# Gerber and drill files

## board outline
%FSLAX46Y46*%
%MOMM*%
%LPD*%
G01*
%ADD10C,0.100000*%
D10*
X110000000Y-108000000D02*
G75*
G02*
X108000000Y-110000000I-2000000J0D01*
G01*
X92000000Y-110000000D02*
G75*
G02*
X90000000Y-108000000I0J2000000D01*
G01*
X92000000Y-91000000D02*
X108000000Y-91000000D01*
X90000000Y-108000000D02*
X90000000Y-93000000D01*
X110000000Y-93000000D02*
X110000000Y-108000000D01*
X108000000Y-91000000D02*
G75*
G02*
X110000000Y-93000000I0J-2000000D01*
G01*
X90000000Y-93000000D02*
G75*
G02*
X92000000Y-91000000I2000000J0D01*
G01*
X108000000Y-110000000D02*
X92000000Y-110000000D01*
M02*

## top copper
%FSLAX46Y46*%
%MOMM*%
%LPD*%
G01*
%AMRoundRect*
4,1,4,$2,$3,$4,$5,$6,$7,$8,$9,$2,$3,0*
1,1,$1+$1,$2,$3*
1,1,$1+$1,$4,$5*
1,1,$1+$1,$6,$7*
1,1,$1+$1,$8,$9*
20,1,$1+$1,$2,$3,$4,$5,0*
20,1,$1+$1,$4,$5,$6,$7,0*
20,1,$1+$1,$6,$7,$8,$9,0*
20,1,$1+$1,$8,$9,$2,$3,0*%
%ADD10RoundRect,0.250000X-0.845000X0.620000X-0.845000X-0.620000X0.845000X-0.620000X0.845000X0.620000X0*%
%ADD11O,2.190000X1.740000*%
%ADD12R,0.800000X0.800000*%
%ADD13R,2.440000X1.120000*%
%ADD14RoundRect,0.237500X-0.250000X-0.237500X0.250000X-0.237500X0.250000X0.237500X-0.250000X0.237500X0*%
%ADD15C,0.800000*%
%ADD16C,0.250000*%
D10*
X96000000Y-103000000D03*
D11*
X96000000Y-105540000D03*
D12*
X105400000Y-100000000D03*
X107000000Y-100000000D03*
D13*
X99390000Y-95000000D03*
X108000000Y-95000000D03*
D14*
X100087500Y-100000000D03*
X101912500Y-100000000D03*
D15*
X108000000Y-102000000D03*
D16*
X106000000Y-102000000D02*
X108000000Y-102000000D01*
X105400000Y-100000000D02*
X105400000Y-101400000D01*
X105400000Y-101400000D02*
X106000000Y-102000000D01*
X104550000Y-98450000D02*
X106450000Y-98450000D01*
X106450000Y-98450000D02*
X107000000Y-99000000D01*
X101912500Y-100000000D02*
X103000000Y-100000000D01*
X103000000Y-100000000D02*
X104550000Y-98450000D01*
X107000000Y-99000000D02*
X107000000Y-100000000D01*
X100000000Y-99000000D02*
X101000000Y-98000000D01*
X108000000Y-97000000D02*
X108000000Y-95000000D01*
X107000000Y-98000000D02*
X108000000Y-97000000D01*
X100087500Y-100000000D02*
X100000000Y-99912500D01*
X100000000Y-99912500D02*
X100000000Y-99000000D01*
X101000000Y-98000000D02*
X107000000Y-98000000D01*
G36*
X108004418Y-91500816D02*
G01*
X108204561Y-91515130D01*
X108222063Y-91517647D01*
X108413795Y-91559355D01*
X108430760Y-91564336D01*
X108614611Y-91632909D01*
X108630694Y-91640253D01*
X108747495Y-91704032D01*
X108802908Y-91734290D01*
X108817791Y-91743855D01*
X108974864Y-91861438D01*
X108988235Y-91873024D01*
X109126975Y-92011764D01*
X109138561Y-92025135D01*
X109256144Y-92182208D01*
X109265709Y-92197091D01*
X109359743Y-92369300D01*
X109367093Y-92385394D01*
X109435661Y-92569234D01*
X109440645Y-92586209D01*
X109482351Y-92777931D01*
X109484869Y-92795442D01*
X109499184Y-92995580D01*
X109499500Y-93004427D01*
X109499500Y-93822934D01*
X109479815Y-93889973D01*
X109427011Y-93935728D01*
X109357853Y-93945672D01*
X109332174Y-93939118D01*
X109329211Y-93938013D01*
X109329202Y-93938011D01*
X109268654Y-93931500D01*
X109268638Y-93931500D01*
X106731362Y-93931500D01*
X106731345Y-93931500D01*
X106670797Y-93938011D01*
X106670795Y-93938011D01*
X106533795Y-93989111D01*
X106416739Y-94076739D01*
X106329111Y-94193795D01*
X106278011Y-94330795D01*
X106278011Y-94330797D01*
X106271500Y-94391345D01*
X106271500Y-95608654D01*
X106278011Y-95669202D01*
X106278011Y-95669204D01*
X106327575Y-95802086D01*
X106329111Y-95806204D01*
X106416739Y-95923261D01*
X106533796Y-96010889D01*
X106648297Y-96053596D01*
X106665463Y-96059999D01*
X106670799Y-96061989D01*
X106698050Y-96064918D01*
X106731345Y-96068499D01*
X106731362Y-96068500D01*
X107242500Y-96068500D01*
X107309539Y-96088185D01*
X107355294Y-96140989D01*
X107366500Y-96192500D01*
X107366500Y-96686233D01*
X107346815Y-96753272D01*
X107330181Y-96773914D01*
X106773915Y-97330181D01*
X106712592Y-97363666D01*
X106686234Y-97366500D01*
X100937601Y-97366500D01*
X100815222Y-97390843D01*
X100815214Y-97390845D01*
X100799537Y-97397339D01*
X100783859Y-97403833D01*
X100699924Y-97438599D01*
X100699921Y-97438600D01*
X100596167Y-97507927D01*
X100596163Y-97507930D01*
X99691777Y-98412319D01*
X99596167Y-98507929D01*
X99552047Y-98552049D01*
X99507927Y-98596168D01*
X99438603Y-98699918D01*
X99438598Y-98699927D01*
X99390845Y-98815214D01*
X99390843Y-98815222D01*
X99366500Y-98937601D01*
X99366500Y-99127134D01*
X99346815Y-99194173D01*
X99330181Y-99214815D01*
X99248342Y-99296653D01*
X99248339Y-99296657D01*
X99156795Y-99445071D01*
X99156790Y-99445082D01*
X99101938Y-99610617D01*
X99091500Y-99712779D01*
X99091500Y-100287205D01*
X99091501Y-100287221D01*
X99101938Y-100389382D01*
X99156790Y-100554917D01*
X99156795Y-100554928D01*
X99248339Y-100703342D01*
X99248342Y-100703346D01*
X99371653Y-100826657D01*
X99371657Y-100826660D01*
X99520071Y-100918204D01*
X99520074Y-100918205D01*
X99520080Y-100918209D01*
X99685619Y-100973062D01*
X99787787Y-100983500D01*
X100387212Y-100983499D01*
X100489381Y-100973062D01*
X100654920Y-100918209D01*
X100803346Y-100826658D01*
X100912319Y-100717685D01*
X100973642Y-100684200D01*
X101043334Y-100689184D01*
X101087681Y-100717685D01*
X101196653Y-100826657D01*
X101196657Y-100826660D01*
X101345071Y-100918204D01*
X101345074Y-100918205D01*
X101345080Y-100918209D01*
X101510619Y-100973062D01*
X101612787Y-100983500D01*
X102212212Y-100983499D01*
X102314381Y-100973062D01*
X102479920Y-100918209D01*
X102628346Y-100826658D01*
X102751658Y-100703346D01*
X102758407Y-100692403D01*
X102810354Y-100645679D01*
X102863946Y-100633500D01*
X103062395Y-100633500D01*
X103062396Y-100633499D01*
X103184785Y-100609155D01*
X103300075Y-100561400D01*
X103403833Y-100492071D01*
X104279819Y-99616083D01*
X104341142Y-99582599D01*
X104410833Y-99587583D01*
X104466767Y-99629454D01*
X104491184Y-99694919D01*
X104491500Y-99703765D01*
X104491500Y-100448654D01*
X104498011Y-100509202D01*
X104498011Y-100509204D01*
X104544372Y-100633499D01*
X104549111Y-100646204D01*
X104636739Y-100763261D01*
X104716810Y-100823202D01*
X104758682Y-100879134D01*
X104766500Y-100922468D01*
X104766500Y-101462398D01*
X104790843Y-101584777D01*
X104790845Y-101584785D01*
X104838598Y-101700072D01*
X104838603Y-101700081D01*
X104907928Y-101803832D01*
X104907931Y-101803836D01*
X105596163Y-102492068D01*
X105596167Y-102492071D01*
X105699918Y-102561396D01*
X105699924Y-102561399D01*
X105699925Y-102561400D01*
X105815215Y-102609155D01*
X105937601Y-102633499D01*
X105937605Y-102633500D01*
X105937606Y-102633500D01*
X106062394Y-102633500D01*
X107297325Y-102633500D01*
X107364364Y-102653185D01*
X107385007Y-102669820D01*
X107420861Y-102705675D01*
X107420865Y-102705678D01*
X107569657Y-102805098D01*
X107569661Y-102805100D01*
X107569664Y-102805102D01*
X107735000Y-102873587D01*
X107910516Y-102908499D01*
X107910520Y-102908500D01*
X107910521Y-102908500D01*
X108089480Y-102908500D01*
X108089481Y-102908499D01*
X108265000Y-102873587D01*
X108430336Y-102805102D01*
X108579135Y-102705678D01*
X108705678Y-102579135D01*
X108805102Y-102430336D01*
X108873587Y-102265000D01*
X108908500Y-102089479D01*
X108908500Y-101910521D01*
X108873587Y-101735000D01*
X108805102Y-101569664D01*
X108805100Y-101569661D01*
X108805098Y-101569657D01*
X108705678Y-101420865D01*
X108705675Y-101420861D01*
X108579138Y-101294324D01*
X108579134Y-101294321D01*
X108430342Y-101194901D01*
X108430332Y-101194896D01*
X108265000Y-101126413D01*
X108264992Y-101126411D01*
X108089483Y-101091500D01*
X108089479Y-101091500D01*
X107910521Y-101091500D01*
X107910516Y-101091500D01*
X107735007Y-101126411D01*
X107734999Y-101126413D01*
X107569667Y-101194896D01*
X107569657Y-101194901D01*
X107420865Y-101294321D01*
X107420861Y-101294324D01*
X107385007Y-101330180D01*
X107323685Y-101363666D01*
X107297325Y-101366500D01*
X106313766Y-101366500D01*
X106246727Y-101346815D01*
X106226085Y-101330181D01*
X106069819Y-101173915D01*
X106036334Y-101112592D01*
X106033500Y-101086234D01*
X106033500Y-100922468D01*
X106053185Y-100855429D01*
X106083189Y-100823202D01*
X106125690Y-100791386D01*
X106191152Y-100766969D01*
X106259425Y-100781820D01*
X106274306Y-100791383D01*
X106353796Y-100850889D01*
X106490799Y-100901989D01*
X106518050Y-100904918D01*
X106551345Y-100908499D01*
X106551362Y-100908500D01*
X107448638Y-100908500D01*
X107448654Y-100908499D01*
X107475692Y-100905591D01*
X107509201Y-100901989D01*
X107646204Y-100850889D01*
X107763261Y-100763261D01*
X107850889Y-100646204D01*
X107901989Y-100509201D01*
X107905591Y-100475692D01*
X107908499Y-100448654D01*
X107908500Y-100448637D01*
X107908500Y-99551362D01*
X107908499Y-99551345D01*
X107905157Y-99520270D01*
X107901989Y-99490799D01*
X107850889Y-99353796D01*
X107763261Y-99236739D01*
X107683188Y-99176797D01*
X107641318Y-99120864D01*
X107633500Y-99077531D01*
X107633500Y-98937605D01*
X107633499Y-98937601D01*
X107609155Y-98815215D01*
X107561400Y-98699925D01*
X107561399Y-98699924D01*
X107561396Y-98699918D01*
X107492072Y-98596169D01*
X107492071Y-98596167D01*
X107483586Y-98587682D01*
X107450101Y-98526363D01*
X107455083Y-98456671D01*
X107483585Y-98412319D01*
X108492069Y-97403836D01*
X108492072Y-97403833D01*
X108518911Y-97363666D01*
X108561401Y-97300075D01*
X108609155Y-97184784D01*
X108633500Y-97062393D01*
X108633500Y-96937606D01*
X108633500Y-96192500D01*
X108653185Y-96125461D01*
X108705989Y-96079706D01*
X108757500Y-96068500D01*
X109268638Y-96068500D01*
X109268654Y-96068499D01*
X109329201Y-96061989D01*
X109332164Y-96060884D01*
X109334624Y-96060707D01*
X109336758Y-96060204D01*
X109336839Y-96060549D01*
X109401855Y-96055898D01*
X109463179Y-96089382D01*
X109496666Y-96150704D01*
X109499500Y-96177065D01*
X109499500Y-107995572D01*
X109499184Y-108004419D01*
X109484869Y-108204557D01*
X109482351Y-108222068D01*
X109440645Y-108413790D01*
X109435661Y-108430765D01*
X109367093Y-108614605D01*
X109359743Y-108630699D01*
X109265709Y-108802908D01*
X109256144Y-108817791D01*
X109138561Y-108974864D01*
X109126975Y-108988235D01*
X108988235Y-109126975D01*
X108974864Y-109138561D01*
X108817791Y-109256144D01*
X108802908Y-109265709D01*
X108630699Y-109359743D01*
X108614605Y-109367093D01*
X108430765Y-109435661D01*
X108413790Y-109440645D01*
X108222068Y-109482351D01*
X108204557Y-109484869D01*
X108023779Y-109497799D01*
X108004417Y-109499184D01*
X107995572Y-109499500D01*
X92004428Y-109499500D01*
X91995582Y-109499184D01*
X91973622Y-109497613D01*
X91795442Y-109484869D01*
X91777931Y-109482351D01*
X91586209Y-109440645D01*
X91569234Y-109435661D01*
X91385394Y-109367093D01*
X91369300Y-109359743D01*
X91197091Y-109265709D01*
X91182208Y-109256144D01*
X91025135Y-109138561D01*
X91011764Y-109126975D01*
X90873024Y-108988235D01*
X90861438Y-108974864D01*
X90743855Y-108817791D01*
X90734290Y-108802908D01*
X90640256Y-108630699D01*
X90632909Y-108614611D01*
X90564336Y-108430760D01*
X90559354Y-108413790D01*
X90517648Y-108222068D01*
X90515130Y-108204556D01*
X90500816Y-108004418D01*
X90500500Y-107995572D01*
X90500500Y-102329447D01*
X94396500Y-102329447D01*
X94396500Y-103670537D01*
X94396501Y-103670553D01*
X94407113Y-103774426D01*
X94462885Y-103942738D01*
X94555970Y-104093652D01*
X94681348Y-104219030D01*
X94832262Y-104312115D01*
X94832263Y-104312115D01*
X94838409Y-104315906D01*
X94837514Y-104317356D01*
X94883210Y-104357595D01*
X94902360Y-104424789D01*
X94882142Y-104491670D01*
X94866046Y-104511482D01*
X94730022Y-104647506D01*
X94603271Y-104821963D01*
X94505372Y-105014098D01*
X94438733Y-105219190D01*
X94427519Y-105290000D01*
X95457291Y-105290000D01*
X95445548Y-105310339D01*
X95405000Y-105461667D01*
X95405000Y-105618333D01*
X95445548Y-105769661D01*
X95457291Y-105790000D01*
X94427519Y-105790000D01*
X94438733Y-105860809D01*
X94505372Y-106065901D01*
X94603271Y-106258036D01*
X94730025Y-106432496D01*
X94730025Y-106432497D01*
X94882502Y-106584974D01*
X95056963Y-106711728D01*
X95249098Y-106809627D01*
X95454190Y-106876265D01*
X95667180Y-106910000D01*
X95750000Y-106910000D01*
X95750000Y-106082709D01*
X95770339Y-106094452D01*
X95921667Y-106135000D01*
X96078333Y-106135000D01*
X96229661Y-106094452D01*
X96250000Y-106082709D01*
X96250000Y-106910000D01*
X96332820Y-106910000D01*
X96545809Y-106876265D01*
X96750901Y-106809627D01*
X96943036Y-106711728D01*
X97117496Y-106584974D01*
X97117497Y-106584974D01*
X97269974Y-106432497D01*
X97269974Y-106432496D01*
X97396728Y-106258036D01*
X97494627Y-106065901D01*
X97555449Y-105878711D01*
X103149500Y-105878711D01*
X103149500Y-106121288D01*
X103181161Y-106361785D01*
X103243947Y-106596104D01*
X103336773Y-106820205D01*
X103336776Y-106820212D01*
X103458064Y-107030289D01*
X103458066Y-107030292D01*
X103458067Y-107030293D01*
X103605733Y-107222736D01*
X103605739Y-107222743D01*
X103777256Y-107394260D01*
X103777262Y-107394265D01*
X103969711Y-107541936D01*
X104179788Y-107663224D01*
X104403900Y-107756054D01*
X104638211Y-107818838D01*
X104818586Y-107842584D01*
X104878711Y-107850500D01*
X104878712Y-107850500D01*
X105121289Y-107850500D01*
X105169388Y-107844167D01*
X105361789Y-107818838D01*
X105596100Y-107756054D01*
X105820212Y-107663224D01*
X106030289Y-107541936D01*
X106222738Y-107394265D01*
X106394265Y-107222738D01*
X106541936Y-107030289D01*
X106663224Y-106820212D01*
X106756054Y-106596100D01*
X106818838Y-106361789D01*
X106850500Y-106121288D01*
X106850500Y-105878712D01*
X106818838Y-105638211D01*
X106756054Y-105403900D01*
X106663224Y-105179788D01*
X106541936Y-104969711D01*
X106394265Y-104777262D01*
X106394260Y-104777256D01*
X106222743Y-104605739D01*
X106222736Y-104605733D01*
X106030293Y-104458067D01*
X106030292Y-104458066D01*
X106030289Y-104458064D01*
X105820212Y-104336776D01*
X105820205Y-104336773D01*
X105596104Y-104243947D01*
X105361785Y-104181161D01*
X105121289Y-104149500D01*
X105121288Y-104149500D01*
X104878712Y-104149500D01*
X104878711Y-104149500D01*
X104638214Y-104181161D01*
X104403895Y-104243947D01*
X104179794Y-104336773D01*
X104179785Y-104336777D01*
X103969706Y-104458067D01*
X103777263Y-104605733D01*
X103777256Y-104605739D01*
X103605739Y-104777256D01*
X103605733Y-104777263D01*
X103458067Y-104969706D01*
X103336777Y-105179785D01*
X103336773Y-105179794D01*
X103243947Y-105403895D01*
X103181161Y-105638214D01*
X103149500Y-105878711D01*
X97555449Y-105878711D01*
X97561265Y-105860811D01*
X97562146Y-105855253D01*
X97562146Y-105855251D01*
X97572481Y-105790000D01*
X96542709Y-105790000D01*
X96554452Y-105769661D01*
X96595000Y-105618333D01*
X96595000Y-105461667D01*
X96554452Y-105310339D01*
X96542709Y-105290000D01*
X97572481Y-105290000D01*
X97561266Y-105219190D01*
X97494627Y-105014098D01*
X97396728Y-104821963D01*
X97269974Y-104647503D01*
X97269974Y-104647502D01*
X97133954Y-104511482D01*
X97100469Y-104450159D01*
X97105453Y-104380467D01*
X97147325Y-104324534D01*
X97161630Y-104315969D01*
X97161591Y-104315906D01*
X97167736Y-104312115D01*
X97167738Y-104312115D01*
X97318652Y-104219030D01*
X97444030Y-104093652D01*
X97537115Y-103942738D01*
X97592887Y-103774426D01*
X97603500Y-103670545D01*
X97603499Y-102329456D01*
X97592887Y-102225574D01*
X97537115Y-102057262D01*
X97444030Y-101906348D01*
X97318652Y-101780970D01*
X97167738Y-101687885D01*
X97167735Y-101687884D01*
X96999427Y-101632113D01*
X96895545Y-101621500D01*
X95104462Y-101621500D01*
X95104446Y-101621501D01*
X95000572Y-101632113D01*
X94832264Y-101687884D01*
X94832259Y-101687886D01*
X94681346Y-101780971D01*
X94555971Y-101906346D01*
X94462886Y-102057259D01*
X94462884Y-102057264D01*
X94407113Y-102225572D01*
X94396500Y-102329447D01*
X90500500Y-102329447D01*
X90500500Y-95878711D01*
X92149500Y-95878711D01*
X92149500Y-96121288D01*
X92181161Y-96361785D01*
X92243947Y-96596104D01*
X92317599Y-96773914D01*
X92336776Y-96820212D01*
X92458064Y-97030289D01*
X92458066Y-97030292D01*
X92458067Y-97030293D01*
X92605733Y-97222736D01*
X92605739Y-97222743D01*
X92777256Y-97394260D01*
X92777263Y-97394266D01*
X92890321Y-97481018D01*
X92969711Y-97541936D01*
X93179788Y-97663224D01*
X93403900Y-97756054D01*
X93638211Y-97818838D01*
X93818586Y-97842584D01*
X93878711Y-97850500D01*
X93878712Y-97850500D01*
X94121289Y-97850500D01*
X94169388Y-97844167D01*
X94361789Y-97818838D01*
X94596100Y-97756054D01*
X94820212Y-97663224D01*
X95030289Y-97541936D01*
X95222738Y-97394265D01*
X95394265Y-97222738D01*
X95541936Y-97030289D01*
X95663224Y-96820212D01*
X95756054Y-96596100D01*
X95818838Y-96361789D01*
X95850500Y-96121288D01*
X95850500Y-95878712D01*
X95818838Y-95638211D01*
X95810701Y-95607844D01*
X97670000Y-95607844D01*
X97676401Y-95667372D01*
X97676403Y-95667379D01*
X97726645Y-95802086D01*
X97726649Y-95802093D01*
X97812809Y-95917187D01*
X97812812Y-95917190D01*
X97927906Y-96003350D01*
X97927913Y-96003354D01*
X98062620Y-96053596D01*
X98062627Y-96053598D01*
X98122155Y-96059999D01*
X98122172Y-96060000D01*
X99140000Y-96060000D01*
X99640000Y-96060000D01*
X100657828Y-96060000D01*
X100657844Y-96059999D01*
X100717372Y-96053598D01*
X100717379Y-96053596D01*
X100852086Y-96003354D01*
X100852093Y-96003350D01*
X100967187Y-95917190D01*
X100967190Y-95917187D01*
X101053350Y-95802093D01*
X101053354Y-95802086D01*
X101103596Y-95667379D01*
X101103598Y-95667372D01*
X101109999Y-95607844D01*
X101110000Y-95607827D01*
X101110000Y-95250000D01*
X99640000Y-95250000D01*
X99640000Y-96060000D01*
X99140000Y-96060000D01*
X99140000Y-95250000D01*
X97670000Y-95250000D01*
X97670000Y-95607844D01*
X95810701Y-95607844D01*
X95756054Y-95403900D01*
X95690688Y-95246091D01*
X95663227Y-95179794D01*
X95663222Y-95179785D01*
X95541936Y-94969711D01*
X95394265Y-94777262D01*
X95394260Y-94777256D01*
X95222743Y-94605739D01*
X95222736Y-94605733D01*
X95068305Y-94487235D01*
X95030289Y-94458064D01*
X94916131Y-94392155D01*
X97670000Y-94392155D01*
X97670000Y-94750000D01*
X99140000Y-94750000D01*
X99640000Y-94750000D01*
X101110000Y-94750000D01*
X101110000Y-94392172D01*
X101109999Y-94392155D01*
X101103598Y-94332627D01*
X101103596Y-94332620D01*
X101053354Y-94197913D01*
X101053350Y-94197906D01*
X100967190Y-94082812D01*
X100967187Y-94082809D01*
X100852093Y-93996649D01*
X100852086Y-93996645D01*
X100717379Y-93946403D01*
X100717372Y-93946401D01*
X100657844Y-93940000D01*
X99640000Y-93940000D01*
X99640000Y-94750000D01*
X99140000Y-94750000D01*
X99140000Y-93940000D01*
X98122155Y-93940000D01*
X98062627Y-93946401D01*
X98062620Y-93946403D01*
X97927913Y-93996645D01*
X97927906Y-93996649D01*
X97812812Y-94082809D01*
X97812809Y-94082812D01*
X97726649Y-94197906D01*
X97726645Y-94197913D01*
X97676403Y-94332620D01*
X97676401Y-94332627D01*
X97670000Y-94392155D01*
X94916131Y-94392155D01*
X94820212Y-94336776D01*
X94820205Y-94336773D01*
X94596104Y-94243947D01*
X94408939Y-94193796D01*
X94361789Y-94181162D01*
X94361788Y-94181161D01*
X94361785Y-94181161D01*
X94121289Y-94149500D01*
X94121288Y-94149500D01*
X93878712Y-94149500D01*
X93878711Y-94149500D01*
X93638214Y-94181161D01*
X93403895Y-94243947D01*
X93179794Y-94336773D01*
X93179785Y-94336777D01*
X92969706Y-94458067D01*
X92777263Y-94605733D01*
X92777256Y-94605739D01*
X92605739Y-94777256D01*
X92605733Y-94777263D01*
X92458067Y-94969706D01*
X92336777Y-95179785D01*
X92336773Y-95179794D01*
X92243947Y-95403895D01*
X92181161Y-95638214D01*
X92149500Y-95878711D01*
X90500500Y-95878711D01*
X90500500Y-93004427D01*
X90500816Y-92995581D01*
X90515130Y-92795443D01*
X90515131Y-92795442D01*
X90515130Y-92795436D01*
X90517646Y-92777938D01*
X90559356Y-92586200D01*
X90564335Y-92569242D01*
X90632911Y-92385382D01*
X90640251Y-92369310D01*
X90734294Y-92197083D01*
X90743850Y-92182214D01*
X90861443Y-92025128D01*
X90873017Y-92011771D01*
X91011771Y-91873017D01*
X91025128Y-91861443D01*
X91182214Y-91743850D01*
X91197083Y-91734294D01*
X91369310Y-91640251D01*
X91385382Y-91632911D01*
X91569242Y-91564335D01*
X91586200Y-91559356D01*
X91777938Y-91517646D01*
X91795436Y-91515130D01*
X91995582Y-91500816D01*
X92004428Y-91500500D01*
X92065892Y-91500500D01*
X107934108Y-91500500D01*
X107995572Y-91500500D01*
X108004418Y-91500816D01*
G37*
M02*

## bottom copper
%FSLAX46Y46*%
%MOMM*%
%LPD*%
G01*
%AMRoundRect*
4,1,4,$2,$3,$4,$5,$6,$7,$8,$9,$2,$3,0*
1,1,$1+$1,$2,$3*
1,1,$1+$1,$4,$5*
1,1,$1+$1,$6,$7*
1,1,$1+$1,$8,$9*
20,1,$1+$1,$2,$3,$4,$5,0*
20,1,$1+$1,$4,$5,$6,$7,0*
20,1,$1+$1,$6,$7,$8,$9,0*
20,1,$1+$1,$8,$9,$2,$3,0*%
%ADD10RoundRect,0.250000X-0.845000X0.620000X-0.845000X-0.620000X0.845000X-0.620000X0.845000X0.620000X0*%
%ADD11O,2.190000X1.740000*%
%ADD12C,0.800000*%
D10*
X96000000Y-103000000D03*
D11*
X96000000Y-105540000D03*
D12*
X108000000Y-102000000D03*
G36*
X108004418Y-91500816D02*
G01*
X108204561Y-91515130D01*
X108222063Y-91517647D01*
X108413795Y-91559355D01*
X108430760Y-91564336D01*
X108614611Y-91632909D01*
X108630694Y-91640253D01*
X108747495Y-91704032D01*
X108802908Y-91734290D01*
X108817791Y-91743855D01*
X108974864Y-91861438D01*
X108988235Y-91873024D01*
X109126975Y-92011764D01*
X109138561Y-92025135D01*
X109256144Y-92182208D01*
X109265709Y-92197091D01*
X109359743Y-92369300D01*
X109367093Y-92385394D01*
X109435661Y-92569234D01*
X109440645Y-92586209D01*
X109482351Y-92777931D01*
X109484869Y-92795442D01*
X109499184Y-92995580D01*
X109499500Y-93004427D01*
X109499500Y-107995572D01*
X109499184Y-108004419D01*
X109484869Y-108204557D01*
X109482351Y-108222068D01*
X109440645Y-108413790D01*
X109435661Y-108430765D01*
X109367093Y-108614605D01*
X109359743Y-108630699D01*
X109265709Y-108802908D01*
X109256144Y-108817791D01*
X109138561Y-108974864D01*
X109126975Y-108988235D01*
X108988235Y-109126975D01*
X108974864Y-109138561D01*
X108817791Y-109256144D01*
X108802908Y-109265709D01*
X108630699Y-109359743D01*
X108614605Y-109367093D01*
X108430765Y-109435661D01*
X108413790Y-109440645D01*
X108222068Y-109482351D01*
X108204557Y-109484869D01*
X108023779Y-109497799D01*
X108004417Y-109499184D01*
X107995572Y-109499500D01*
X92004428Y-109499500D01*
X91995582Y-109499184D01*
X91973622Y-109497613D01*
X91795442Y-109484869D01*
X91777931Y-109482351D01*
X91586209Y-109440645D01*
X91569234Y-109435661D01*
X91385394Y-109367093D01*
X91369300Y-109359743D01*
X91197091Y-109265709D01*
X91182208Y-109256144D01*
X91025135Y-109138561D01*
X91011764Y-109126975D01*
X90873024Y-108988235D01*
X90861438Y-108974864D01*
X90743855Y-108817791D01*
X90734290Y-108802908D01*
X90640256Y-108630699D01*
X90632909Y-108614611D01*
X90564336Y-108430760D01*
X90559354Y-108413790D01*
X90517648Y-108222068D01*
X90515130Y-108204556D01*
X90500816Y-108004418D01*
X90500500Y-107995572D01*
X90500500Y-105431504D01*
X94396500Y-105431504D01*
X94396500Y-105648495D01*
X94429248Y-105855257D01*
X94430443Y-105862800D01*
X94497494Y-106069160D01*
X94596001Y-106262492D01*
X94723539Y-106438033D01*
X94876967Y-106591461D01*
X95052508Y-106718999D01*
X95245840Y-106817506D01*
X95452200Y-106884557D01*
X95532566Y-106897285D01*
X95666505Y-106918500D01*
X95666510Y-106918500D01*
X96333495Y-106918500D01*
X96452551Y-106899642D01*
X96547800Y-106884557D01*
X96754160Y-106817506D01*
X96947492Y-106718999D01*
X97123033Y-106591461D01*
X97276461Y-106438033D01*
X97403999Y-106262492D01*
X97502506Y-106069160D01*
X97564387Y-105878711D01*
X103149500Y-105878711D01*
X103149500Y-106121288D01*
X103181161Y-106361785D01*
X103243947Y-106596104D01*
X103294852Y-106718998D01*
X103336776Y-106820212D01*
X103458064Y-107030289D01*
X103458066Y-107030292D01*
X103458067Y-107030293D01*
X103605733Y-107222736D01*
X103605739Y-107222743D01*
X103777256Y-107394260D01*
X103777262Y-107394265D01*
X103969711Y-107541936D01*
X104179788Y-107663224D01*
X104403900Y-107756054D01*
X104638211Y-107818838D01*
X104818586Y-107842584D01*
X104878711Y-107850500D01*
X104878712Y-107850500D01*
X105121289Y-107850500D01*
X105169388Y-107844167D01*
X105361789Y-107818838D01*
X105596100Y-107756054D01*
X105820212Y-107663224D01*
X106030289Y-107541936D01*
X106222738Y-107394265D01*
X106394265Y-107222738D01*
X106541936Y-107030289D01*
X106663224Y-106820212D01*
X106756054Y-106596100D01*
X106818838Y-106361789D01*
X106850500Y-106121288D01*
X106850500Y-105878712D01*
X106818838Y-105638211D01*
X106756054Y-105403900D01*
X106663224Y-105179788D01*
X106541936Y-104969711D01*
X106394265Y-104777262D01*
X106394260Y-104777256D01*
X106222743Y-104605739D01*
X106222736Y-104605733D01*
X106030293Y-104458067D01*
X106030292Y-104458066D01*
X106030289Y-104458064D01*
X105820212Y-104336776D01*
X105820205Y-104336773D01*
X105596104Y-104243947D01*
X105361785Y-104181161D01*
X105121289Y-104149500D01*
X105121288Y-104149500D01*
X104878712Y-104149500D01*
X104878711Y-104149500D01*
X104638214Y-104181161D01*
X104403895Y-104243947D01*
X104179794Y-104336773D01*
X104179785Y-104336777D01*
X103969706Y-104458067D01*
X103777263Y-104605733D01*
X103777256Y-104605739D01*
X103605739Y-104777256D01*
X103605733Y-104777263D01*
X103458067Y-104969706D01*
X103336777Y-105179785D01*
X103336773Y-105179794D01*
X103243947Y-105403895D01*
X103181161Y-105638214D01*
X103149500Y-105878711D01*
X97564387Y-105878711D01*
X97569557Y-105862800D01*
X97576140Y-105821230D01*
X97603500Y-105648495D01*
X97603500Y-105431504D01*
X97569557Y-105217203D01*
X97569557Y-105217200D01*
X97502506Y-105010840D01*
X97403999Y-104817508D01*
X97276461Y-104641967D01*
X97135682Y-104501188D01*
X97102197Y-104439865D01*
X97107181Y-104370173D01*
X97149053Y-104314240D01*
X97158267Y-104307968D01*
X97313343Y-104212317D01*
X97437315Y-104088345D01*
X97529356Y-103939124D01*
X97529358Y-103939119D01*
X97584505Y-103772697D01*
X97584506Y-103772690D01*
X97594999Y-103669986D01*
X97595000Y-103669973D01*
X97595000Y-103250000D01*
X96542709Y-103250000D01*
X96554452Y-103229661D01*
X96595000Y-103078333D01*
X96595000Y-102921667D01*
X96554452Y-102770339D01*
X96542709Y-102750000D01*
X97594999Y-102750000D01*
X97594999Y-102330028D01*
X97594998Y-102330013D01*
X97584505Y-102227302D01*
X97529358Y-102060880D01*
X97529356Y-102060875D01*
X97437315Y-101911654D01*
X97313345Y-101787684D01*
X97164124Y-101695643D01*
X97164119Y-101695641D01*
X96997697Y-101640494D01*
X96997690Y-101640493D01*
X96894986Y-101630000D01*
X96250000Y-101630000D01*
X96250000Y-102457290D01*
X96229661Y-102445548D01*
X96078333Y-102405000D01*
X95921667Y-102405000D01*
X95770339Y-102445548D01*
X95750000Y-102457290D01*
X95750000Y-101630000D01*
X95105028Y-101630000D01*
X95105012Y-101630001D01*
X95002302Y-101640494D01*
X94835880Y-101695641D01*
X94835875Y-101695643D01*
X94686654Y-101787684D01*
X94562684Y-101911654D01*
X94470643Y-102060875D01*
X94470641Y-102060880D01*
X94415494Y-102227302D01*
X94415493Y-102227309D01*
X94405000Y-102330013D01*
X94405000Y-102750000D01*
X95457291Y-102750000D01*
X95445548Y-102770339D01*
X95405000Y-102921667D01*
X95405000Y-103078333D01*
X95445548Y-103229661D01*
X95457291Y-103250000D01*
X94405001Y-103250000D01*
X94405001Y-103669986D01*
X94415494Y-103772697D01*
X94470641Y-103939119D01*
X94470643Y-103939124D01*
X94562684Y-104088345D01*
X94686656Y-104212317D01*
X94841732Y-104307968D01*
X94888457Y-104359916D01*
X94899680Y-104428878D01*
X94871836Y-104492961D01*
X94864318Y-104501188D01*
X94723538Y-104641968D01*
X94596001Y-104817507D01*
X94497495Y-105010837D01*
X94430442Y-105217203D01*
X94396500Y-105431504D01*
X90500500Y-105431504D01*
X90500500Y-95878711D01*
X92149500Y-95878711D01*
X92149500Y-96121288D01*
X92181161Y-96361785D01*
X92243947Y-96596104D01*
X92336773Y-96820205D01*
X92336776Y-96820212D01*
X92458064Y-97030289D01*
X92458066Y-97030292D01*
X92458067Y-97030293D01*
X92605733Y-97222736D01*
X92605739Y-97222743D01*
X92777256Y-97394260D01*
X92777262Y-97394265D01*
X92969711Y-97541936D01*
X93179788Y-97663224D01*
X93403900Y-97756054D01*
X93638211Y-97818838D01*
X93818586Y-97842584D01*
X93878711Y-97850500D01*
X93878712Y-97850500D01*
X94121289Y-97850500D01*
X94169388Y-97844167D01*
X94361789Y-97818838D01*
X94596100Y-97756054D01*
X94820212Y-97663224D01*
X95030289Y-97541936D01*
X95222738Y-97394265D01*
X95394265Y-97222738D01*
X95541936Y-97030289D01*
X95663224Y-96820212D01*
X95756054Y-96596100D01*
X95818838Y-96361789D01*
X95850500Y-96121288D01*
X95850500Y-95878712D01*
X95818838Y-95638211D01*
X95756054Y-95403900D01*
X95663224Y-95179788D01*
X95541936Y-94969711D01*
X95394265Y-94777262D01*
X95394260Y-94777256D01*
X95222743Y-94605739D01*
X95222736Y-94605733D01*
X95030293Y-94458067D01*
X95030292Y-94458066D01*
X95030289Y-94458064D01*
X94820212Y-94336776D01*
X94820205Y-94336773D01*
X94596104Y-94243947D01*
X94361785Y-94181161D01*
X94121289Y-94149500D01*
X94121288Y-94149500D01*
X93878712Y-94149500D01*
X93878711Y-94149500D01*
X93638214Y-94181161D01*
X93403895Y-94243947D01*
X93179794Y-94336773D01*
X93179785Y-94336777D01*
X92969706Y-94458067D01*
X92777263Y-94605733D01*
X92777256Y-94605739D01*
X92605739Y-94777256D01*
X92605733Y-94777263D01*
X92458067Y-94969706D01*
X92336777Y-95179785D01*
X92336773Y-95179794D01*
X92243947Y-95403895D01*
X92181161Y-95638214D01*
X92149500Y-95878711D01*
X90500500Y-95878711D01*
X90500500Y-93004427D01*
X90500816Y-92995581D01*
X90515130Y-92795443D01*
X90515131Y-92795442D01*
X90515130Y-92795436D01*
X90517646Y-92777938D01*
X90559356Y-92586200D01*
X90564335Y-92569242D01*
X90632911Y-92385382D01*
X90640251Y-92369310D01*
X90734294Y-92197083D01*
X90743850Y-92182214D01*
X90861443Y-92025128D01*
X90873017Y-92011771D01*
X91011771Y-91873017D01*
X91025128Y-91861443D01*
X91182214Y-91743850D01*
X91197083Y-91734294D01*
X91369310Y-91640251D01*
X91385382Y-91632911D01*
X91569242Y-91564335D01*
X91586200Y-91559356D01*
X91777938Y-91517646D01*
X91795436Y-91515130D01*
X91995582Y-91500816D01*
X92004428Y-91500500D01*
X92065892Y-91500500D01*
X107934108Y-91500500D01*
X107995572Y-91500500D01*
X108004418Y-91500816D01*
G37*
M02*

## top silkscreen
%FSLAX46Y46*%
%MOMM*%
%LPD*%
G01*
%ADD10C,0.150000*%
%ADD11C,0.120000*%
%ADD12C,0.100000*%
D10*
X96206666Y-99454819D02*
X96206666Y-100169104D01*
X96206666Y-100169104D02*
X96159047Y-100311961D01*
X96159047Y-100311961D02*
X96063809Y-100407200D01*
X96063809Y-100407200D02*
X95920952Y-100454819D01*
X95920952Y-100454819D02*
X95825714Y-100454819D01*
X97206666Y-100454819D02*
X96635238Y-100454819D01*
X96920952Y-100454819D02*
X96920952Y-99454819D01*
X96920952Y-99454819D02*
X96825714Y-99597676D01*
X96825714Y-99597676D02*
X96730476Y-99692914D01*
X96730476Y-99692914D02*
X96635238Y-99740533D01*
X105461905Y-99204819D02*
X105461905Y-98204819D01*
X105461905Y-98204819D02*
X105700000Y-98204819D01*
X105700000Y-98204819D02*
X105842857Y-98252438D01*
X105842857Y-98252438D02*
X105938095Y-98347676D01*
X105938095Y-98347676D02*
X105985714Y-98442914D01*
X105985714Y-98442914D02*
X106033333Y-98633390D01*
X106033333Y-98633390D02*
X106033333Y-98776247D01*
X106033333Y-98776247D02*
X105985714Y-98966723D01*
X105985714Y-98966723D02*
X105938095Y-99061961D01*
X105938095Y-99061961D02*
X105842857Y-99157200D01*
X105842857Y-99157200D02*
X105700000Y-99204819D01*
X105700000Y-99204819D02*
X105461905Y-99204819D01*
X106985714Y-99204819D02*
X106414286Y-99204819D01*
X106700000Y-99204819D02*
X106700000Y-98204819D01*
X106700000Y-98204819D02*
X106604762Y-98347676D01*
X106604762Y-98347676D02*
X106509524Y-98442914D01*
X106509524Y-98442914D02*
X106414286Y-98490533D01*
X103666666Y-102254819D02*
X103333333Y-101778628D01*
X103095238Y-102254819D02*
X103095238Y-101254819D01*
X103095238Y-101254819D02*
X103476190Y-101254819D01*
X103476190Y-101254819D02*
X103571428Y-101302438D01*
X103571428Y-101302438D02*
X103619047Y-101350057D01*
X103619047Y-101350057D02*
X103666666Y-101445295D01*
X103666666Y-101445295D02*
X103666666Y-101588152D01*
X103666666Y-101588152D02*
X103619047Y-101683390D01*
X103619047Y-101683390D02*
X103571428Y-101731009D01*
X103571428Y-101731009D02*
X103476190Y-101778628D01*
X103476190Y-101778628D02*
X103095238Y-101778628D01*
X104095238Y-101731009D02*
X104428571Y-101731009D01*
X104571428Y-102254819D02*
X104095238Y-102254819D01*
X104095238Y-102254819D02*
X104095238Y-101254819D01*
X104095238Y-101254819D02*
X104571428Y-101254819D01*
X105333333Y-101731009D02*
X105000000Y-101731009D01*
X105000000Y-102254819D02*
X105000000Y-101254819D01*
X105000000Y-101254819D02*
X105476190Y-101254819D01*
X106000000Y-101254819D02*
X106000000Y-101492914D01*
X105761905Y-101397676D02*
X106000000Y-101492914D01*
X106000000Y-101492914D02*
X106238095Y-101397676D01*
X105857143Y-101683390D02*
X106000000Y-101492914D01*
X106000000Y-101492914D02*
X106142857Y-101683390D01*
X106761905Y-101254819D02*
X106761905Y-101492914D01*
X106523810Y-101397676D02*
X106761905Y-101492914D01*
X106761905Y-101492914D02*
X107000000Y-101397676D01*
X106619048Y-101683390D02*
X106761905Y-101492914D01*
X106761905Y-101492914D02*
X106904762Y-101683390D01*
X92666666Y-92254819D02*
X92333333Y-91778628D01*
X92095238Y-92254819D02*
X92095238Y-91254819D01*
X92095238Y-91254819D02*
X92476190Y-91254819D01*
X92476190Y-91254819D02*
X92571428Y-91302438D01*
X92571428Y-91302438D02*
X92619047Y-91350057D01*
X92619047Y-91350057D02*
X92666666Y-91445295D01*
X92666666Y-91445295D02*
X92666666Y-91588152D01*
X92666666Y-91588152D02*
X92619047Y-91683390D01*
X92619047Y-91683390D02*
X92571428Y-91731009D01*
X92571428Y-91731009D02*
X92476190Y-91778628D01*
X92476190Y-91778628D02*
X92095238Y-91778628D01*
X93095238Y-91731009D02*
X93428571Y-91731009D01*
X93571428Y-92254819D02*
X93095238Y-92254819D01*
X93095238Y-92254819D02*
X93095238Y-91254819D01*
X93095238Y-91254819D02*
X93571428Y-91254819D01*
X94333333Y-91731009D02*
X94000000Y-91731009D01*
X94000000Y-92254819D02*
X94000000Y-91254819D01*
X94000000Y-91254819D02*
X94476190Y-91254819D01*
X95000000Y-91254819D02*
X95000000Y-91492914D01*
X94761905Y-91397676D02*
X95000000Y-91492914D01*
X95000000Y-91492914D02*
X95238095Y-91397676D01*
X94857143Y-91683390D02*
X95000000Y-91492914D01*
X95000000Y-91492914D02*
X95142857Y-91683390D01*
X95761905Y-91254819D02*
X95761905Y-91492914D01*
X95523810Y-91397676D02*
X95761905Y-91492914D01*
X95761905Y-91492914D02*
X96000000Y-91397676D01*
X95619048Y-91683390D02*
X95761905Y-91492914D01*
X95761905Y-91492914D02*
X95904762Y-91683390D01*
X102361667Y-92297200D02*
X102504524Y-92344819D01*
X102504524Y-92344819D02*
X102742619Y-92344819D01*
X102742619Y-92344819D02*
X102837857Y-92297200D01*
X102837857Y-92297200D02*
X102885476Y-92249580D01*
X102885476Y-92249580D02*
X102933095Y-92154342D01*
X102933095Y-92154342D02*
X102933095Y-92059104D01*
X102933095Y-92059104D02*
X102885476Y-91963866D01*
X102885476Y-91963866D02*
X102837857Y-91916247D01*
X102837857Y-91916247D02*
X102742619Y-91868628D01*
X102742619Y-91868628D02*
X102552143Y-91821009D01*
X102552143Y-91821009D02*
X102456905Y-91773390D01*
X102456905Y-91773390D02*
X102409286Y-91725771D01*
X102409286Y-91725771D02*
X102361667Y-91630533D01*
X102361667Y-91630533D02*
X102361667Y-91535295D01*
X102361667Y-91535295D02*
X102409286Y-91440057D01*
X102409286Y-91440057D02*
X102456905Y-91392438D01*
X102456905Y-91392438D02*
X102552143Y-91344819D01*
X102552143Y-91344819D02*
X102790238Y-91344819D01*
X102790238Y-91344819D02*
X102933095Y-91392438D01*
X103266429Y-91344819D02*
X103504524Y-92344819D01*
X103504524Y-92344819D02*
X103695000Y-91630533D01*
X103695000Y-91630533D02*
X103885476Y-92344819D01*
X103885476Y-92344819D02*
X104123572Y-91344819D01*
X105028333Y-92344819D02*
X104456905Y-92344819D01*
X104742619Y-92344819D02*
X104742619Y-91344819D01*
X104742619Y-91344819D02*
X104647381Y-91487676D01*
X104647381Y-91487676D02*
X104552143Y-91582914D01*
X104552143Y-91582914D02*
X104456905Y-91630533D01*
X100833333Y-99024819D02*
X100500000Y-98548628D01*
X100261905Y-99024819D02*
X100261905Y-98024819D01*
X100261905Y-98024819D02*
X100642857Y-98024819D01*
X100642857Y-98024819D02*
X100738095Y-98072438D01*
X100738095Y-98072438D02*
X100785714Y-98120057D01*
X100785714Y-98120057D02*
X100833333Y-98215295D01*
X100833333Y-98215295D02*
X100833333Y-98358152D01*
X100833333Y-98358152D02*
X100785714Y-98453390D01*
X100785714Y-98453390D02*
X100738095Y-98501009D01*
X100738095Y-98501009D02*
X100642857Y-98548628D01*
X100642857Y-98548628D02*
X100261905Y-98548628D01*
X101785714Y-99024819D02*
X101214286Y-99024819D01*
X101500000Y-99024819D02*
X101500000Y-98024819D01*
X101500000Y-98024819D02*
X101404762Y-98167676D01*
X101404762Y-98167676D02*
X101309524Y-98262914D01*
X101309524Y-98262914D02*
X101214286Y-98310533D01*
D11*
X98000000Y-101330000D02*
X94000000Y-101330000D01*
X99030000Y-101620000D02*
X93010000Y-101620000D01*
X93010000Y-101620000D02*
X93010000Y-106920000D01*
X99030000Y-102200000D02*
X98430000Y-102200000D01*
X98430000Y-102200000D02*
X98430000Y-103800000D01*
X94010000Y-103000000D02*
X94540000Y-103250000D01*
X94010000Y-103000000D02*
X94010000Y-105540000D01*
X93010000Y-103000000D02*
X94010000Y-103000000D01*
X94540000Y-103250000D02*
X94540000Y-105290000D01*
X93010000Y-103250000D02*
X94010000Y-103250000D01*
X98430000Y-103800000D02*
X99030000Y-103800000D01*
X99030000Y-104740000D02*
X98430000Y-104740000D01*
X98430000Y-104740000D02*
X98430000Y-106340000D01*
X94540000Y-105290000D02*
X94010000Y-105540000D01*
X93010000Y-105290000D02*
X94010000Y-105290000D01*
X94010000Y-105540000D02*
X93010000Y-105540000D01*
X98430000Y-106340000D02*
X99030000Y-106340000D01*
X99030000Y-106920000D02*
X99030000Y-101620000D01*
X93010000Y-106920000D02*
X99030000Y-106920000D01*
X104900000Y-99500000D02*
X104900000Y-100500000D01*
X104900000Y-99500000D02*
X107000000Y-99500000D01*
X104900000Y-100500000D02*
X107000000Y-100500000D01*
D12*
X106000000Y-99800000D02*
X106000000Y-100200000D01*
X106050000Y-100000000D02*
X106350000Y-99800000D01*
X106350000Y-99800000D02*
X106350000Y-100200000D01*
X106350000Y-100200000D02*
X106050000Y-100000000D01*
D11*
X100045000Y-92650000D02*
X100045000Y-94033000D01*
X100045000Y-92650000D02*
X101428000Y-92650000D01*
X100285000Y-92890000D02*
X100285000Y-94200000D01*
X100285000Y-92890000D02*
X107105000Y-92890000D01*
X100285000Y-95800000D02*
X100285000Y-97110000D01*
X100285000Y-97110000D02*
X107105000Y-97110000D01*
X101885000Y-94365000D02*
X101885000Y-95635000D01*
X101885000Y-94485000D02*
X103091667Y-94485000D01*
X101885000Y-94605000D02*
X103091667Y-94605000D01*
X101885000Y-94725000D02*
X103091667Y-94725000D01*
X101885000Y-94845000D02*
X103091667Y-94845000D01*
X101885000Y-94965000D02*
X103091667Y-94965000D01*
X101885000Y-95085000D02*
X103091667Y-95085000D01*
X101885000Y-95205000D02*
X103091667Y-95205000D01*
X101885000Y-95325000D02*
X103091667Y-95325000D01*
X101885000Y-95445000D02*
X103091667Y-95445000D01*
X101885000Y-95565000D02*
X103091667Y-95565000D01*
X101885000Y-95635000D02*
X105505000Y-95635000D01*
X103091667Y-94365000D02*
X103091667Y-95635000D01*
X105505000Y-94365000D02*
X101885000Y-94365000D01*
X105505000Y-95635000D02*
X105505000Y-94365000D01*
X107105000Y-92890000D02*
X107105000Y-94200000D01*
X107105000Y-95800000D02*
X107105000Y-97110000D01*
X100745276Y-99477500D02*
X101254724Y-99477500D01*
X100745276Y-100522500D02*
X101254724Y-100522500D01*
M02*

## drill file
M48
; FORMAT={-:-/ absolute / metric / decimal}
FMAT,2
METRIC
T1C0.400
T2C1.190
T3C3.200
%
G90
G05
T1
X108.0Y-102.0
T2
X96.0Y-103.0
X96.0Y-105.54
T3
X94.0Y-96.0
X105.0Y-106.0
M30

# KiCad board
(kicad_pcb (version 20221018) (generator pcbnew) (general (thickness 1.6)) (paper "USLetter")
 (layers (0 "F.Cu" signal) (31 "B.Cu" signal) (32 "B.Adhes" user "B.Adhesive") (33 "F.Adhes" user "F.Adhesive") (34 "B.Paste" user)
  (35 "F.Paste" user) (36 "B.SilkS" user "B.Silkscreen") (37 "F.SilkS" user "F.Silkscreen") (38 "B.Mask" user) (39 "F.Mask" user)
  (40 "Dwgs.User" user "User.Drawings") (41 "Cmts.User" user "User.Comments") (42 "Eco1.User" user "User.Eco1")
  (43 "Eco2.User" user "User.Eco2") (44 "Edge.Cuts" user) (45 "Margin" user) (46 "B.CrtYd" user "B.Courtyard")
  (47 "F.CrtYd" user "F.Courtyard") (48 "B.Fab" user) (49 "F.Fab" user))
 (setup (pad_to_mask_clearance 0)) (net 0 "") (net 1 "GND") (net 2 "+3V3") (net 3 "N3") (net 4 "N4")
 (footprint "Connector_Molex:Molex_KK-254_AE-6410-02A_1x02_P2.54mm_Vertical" (layer "F.Cu") (at 96 103 -90)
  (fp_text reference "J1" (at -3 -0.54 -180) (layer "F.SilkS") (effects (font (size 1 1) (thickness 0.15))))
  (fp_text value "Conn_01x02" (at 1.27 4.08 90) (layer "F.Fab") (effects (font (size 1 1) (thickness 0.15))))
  (fp_line (start -1.67 -2) (end -1.67 2) (stroke (width 0.12) (type solid)) (layer "F.SilkS"))
  (fp_line (start -1.38 -3.03) (end -1.38 2.99) (stroke (width 0.12) (type solid)) (layer "F.SilkS"))
  (fp_line (start -1.38 2.99) (end 3.92 2.99) (stroke (width 0.12) (type solid)) (layer "F.SilkS"))
  (fp_line (start -0.8 -3.03) (end -0.8 -2.43) (stroke (width 0.12) (type solid)) (layer "F.SilkS"))
  (fp_line (start -0.8 -2.43) (end 0.8 -2.43) (stroke (width 0.12) (type solid)) (layer "F.SilkS"))
  (fp_line (start 0 1.99) (end 0.25 1.46) (stroke (width 0.12) (type solid)) (layer "F.SilkS"))
  (fp_line (start 0 1.99) (end 2.54 1.99) (stroke (width 0.12) (type solid)) (layer "F.SilkS"))
  (fp_line (start 0 2.99) (end 0 1.99) (stroke (width 0.12) (type solid)) (layer "F.SilkS"))
  (fp_line (start 0.25 1.46) (end 2.29 1.46) (stroke (width 0.12) (type solid)) (layer "F.SilkS"))
  (fp_line (start 0.25 2.99) (end 0.25 1.99) (stroke (width 0.12) (type solid)) (layer "F.SilkS"))
  (fp_line (start 0.8 -2.43) (end 0.8 -3.03) (stroke (width 0.12) (type solid)) (layer "F.SilkS"))
  (fp_line (start 1.74 -3.03) (end 1.74 -2.43) (stroke (width 0.12) (type solid)) (layer "F.SilkS"))
  (fp_line (start 1.74 -2.43) (end 3.34 -2.43) (stroke (width 0.12) (type solid)) (layer "F.SilkS"))
  (fp_line (start 2.29 1.46) (end 2.54 1.99) (stroke (width 0.12) (type solid)) (layer "F.SilkS"))
  (fp_line (start 2.29 2.99) (end 2.29 1.99) (stroke (width 0.12) (type solid)) (layer "F.SilkS"))
  (fp_line (start 2.54 1.99) (end 2.54 2.99) (stroke (width 0.12) (type solid)) (layer "F.SilkS"))
  (fp_line (start 3.34 -2.43) (end 3.34 -3.03) (stroke (width 0.12) (type solid)) (layer "F.SilkS"))
  (fp_line (start 3.92 -3.03) (end -1.38 -3.03) (stroke (width 0.12) (type solid)) (layer "F.SilkS"))
  (fp_line (start 3.92 2.99) (end 3.92 -3.03) (stroke (width 0.12) (type solid)) (layer "F.SilkS"))
  (pad "1" thru_hole roundrect (at 0 0 270) (size 1.74 2.19) (drill 1.19) (layers "*.Cu" "*.Mask") (roundrect_rratio 0.143678) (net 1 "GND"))
  (pad "2" thru_hole oval (at 2.54 0 270) (size 1.74 2.19) (drill 1.19) (layers "*.Cu" "*.Mask") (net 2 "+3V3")))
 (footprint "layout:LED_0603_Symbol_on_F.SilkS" (layer "F.Cu") (at 106.2 100)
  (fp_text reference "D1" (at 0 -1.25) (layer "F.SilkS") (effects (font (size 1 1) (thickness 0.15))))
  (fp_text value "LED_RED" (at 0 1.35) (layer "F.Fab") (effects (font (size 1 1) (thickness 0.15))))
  (fp_line (start -1.3 -0.5) (end -1.3 0.5) (stroke (width 0.12) (type solid)) (layer "F.SilkS"))
  (fp_line (start -1.3 -0.5) (end 0.8 -0.5) (stroke (width 0.12) (type solid)) (layer "F.SilkS"))
  (fp_line (start -1.3 0.5) (end 0.8 0.5) (stroke (width 0.12) (type solid)) (layer "F.SilkS"))
  (fp_line (start -0.2 -0.2) (end -0.2 0.2) (stroke (width 0.1) (type solid)) (layer "F.SilkS"))
  (fp_line (start -0.15 0) (end 0.15 -0.2) (stroke (width 0.1) (type solid)) (layer "F.SilkS"))
  (fp_line (start 0.15 -0.2) (end 0.15 0.2) (stroke (width 0.1) (type solid)) (layer "F.SilkS"))
  (fp_line (start 0.15 0.2) (end -0.15 0) (stroke (width 0.1) (type solid)) (layer "F.SilkS"))
  (pad "1" smd rect (at -0.8 0 180) (size 0.8 0.8) (layers "F.Cu" "F.Paste" "F.Mask") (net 1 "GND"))
  (pad "2" smd rect (at 0.8 0 180) (size 0.8 0.8) (layers "F.Cu" "F.Paste" "F.Mask") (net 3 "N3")))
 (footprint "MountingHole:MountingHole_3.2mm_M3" (layer "F.Cu") (at 105 106)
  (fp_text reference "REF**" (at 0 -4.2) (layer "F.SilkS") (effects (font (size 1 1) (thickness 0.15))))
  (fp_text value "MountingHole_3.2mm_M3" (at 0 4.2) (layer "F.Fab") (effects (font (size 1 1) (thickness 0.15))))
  (pad "" np_thru_hole circle (at 0 0) (size 3.2 3.2) (drill 3.2) (layers "F&B.Cu" "*.Mask")))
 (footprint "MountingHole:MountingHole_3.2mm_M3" (layer "F.Cu") (at 94 96)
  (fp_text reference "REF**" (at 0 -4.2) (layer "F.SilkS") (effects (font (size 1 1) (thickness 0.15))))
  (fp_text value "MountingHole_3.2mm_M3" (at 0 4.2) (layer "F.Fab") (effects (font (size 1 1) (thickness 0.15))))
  (pad "" np_thru_hole circle (at 0 0) (size 3.2 3.2) (drill 3.2) (layers "*.Cu" "*.Mask")))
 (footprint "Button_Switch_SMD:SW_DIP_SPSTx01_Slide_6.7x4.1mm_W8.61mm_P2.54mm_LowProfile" (layer "F.Cu") (at 103.695 95)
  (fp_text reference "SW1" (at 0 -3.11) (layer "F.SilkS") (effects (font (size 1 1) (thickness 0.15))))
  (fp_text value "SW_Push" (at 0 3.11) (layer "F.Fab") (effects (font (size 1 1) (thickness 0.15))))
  (fp_line (start -3.65 -2.35) (end -3.65 -0.967) (stroke (width 0.12) (type solid)) (layer "F.SilkS"))
  (fp_line (start -3.65 -2.35) (end -2.267 -2.35) (stroke (width 0.12) (type solid)) (layer "F.SilkS"))
  (fp_line (start -3.41 -2.11) (end -3.41 -0.8) (stroke (width 0.12) (type solid)) (layer "F.SilkS"))
  (fp_line (start -3.41 -2.11) (end 3.41 -2.11) (stroke (width 0.12) (type solid)) (layer "F.SilkS"))
  (fp_line (start -3.41 0.8) (end -3.41 2.11) (stroke (width 0.12) (type solid)) (layer "F.SilkS"))
  (fp_line (start -3.41 2.11) (end 3.41 2.11) (stroke (width 0.12) (type solid)) (layer "F.SilkS"))
  (fp_line (start -1.81 -0.635) (end -1.81 0.635) (stroke (width 0.12) (type solid)) (layer "F.SilkS"))
  (fp_line (start -1.81 -0.515) (end -0.603333 -0.515) (stroke (width 0.12) (type solid)) (layer "F.SilkS"))
  (fp_line (start -1.81 -0.395) (end -0.603333 -0.395) (stroke (width 0.12) (type solid)) (layer "F.SilkS"))
  (fp_line (start -1.81 -0.275) (end -0.603333 -0.275) (stroke (width 0.12) (type solid)) (layer "F.SilkS"))
  (fp_line (start -1.81 -0.155) (end -0.603333 -0.155) (stroke (width 0.12) (type solid)) (layer "F.SilkS"))
  (fp_line (start -1.81 -0.035) (end -0.603333 -0.035) (stroke (width 0.12) (type solid)) (layer "F.SilkS"))
  (fp_line (start -1.81 0.085) (end -0.603333 0.085) (stroke (width 0.12) (type solid)) (layer "F.SilkS"))
  (fp_line (start -1.81 0.205) (end -0.603333 0.205) (stroke (width 0.12) (type solid)) (layer "F.SilkS"))
  (fp_line (start -1.81 0.325) (end -0.603333 0.325) (stroke (width 0.12) (type solid)) (layer "F.SilkS"))
  (fp_line (start -1.81 0.445) (end -0.603333 0.445) (stroke (width 0.12) (type solid)) (layer "F.SilkS"))
  (fp_line (start -1.81 0.565) (end -0.603333 0.565) (stroke (width 0.12) (type solid)) (layer "F.SilkS"))
  (fp_line (start -1.81 0.635) (end 1.81 0.635) (stroke (width 0.12) (type solid)) (layer "F.SilkS"))
  (fp_line (start -0.603333 -0.635) (end -0.603333 0.635) (stroke (width 0.12) (type solid)) (layer "F.SilkS"))
  (fp_line (start 1.81 -0.635) (end -1.81 -0.635) (stroke (width 0.12) (type solid)) (layer "F.SilkS"))
  (fp_line (start 1.81 0.635) (end 1.81 -0.635) (stroke (width 0.12) (type solid)) (layer "F.SilkS"))
  (fp_line (start 3.41 -2.11) (end 3.41 -0.8) (stroke (width 0.12) (type solid)) (layer "F.SilkS"))
  (fp_line (start 3.41 0.8) (end 3.41 2.11) (stroke (width 0.12) (type solid)) (layer "F.SilkS"))
  (pad "1" smd rect (at -4.305 0) (size 2.44 1.12) (layers "F.Cu" "F.Paste" "F.Mask") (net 2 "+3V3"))
  (pad "2" smd rect (at 4.305 0) (size 2.44 1.12) (layers "F.Cu" "F.Paste" "F.Mask") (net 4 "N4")))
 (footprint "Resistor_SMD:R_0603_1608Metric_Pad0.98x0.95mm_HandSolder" (layer "F.Cu") (at 101 100)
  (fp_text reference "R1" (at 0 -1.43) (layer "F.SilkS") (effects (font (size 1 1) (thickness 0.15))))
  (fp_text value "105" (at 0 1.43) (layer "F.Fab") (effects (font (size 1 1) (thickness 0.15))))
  (fp_line (start -0.254724 -0.5225) (end 0.254724 -0.5225) (stroke (width 0.12) (type solid)) (layer "F.SilkS"))
  (fp_line (start -0.254724 0.5225) (end 0.254724 0.5225) (stroke (width 0.12) (type solid)) (layer "F.SilkS"))
  (pad "1" smd roundrect (at -0.9125 0) (size 0.975 0.95) (layers "F.Cu" "F.Paste" "F.Mask") (roundrect_rratio 0.25) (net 4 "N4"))
  (pad "2" smd roundrect (at 0.9125 0) (size 0.975 0.95) (layers "F.Cu" "F.Paste" "F.Mask") (roundrect_rratio 0.25) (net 3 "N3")))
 (gr_arc (start 110 108) (mid 109.414214 109.414214) (end 108 110) (stroke (width 0.1) (type default)) (layer "Edge.Cuts"))
 (gr_arc (start 92 110) (mid 90.585786 109.414214) (end 90 108) (stroke (width 0.1) (type default)) (layer "Edge.Cuts"))
 (gr_line (start 92 91) (end 108 91) (stroke (width 0.1) (type default)) (layer "Edge.Cuts"))
 (gr_line (start 90 108) (end 90 93) (stroke (width 0.1) (type default)) (layer "Edge.Cuts"))
 (gr_line (start 110 93) (end 110 108) (stroke (width 0.1) (type default)) (layer "Edge.Cuts"))
 (gr_arc (start 108 91) (mid 109.414214 91.585786) (end 110 93) (stroke (width 0.1) (type default)) (layer "Edge.Cuts"))
 (gr_arc (start 90 93) (mid 90.585786 91.585786) (end 92 91) (stroke (width 0.1) (type default)) (layer "Edge.Cuts"))
 (gr_line (start 108 110) (end 92 110) (stroke (width 0.1) (type default)) (layer "Edge.Cuts"))
 (segment (start 106 102) (end 108 102) (width 0.25) (layer "F.Cu") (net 1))
 (segment (start 105.4 100) (end 105.4 101.4) (width 0.25) (layer "F.Cu") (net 1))
 (segment (start 105.4 101.4) (end 106 102) (width 0.25) (layer "F.Cu") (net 1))
 (via (at 108 102) (size 0.8) (drill 0.4) (layers "F.Cu" "B.Cu") (free) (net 1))
 (segment (start 104.55 98.45) (end 106.45 98.45) (width 0.25) (layer "F.Cu") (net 3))
 (segment (start 106.45 98.45) (end 107 99) (width 0.25) (layer "F.Cu") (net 3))
 (segment (start 101.9125 100) (end 103 100) (width 0.25) (layer "F.Cu") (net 3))
 (segment (start 103 100) (end 104.55 98.45) (width 0.25) (layer "F.Cu") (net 3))
 (segment (start 107 99) (end 107 100) (width 0.25) (layer "F.Cu") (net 3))
 (segment (start 100 99) (end 101 98) (width 0.25) (layer "F.Cu") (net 4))
 (segment (start 108 97) (end 108 95) (width 0.25) (layer "F.Cu") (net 4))
 (segment (start 107 98) (end 108 97) (width 0.25) (layer "F.Cu") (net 4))
 (segment (start 100.0875 100) (end 100 99.9125) (width 0.25) (layer "F.Cu") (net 4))
 (segment (start 100 99.9125) (end 100 99) (width 0.25) (layer "F.Cu") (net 4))
 (segment (start 101 98) (end 107 98) (width 0.25) (layer "F.Cu") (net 4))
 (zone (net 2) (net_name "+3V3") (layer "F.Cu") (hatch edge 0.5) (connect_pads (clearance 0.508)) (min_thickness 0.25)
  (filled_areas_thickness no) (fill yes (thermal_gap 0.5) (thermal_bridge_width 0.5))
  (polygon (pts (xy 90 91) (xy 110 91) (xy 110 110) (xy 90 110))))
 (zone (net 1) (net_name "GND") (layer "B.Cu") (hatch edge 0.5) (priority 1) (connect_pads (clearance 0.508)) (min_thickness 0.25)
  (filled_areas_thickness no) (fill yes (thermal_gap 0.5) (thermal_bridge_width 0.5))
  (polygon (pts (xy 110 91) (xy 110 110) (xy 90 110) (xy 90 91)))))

